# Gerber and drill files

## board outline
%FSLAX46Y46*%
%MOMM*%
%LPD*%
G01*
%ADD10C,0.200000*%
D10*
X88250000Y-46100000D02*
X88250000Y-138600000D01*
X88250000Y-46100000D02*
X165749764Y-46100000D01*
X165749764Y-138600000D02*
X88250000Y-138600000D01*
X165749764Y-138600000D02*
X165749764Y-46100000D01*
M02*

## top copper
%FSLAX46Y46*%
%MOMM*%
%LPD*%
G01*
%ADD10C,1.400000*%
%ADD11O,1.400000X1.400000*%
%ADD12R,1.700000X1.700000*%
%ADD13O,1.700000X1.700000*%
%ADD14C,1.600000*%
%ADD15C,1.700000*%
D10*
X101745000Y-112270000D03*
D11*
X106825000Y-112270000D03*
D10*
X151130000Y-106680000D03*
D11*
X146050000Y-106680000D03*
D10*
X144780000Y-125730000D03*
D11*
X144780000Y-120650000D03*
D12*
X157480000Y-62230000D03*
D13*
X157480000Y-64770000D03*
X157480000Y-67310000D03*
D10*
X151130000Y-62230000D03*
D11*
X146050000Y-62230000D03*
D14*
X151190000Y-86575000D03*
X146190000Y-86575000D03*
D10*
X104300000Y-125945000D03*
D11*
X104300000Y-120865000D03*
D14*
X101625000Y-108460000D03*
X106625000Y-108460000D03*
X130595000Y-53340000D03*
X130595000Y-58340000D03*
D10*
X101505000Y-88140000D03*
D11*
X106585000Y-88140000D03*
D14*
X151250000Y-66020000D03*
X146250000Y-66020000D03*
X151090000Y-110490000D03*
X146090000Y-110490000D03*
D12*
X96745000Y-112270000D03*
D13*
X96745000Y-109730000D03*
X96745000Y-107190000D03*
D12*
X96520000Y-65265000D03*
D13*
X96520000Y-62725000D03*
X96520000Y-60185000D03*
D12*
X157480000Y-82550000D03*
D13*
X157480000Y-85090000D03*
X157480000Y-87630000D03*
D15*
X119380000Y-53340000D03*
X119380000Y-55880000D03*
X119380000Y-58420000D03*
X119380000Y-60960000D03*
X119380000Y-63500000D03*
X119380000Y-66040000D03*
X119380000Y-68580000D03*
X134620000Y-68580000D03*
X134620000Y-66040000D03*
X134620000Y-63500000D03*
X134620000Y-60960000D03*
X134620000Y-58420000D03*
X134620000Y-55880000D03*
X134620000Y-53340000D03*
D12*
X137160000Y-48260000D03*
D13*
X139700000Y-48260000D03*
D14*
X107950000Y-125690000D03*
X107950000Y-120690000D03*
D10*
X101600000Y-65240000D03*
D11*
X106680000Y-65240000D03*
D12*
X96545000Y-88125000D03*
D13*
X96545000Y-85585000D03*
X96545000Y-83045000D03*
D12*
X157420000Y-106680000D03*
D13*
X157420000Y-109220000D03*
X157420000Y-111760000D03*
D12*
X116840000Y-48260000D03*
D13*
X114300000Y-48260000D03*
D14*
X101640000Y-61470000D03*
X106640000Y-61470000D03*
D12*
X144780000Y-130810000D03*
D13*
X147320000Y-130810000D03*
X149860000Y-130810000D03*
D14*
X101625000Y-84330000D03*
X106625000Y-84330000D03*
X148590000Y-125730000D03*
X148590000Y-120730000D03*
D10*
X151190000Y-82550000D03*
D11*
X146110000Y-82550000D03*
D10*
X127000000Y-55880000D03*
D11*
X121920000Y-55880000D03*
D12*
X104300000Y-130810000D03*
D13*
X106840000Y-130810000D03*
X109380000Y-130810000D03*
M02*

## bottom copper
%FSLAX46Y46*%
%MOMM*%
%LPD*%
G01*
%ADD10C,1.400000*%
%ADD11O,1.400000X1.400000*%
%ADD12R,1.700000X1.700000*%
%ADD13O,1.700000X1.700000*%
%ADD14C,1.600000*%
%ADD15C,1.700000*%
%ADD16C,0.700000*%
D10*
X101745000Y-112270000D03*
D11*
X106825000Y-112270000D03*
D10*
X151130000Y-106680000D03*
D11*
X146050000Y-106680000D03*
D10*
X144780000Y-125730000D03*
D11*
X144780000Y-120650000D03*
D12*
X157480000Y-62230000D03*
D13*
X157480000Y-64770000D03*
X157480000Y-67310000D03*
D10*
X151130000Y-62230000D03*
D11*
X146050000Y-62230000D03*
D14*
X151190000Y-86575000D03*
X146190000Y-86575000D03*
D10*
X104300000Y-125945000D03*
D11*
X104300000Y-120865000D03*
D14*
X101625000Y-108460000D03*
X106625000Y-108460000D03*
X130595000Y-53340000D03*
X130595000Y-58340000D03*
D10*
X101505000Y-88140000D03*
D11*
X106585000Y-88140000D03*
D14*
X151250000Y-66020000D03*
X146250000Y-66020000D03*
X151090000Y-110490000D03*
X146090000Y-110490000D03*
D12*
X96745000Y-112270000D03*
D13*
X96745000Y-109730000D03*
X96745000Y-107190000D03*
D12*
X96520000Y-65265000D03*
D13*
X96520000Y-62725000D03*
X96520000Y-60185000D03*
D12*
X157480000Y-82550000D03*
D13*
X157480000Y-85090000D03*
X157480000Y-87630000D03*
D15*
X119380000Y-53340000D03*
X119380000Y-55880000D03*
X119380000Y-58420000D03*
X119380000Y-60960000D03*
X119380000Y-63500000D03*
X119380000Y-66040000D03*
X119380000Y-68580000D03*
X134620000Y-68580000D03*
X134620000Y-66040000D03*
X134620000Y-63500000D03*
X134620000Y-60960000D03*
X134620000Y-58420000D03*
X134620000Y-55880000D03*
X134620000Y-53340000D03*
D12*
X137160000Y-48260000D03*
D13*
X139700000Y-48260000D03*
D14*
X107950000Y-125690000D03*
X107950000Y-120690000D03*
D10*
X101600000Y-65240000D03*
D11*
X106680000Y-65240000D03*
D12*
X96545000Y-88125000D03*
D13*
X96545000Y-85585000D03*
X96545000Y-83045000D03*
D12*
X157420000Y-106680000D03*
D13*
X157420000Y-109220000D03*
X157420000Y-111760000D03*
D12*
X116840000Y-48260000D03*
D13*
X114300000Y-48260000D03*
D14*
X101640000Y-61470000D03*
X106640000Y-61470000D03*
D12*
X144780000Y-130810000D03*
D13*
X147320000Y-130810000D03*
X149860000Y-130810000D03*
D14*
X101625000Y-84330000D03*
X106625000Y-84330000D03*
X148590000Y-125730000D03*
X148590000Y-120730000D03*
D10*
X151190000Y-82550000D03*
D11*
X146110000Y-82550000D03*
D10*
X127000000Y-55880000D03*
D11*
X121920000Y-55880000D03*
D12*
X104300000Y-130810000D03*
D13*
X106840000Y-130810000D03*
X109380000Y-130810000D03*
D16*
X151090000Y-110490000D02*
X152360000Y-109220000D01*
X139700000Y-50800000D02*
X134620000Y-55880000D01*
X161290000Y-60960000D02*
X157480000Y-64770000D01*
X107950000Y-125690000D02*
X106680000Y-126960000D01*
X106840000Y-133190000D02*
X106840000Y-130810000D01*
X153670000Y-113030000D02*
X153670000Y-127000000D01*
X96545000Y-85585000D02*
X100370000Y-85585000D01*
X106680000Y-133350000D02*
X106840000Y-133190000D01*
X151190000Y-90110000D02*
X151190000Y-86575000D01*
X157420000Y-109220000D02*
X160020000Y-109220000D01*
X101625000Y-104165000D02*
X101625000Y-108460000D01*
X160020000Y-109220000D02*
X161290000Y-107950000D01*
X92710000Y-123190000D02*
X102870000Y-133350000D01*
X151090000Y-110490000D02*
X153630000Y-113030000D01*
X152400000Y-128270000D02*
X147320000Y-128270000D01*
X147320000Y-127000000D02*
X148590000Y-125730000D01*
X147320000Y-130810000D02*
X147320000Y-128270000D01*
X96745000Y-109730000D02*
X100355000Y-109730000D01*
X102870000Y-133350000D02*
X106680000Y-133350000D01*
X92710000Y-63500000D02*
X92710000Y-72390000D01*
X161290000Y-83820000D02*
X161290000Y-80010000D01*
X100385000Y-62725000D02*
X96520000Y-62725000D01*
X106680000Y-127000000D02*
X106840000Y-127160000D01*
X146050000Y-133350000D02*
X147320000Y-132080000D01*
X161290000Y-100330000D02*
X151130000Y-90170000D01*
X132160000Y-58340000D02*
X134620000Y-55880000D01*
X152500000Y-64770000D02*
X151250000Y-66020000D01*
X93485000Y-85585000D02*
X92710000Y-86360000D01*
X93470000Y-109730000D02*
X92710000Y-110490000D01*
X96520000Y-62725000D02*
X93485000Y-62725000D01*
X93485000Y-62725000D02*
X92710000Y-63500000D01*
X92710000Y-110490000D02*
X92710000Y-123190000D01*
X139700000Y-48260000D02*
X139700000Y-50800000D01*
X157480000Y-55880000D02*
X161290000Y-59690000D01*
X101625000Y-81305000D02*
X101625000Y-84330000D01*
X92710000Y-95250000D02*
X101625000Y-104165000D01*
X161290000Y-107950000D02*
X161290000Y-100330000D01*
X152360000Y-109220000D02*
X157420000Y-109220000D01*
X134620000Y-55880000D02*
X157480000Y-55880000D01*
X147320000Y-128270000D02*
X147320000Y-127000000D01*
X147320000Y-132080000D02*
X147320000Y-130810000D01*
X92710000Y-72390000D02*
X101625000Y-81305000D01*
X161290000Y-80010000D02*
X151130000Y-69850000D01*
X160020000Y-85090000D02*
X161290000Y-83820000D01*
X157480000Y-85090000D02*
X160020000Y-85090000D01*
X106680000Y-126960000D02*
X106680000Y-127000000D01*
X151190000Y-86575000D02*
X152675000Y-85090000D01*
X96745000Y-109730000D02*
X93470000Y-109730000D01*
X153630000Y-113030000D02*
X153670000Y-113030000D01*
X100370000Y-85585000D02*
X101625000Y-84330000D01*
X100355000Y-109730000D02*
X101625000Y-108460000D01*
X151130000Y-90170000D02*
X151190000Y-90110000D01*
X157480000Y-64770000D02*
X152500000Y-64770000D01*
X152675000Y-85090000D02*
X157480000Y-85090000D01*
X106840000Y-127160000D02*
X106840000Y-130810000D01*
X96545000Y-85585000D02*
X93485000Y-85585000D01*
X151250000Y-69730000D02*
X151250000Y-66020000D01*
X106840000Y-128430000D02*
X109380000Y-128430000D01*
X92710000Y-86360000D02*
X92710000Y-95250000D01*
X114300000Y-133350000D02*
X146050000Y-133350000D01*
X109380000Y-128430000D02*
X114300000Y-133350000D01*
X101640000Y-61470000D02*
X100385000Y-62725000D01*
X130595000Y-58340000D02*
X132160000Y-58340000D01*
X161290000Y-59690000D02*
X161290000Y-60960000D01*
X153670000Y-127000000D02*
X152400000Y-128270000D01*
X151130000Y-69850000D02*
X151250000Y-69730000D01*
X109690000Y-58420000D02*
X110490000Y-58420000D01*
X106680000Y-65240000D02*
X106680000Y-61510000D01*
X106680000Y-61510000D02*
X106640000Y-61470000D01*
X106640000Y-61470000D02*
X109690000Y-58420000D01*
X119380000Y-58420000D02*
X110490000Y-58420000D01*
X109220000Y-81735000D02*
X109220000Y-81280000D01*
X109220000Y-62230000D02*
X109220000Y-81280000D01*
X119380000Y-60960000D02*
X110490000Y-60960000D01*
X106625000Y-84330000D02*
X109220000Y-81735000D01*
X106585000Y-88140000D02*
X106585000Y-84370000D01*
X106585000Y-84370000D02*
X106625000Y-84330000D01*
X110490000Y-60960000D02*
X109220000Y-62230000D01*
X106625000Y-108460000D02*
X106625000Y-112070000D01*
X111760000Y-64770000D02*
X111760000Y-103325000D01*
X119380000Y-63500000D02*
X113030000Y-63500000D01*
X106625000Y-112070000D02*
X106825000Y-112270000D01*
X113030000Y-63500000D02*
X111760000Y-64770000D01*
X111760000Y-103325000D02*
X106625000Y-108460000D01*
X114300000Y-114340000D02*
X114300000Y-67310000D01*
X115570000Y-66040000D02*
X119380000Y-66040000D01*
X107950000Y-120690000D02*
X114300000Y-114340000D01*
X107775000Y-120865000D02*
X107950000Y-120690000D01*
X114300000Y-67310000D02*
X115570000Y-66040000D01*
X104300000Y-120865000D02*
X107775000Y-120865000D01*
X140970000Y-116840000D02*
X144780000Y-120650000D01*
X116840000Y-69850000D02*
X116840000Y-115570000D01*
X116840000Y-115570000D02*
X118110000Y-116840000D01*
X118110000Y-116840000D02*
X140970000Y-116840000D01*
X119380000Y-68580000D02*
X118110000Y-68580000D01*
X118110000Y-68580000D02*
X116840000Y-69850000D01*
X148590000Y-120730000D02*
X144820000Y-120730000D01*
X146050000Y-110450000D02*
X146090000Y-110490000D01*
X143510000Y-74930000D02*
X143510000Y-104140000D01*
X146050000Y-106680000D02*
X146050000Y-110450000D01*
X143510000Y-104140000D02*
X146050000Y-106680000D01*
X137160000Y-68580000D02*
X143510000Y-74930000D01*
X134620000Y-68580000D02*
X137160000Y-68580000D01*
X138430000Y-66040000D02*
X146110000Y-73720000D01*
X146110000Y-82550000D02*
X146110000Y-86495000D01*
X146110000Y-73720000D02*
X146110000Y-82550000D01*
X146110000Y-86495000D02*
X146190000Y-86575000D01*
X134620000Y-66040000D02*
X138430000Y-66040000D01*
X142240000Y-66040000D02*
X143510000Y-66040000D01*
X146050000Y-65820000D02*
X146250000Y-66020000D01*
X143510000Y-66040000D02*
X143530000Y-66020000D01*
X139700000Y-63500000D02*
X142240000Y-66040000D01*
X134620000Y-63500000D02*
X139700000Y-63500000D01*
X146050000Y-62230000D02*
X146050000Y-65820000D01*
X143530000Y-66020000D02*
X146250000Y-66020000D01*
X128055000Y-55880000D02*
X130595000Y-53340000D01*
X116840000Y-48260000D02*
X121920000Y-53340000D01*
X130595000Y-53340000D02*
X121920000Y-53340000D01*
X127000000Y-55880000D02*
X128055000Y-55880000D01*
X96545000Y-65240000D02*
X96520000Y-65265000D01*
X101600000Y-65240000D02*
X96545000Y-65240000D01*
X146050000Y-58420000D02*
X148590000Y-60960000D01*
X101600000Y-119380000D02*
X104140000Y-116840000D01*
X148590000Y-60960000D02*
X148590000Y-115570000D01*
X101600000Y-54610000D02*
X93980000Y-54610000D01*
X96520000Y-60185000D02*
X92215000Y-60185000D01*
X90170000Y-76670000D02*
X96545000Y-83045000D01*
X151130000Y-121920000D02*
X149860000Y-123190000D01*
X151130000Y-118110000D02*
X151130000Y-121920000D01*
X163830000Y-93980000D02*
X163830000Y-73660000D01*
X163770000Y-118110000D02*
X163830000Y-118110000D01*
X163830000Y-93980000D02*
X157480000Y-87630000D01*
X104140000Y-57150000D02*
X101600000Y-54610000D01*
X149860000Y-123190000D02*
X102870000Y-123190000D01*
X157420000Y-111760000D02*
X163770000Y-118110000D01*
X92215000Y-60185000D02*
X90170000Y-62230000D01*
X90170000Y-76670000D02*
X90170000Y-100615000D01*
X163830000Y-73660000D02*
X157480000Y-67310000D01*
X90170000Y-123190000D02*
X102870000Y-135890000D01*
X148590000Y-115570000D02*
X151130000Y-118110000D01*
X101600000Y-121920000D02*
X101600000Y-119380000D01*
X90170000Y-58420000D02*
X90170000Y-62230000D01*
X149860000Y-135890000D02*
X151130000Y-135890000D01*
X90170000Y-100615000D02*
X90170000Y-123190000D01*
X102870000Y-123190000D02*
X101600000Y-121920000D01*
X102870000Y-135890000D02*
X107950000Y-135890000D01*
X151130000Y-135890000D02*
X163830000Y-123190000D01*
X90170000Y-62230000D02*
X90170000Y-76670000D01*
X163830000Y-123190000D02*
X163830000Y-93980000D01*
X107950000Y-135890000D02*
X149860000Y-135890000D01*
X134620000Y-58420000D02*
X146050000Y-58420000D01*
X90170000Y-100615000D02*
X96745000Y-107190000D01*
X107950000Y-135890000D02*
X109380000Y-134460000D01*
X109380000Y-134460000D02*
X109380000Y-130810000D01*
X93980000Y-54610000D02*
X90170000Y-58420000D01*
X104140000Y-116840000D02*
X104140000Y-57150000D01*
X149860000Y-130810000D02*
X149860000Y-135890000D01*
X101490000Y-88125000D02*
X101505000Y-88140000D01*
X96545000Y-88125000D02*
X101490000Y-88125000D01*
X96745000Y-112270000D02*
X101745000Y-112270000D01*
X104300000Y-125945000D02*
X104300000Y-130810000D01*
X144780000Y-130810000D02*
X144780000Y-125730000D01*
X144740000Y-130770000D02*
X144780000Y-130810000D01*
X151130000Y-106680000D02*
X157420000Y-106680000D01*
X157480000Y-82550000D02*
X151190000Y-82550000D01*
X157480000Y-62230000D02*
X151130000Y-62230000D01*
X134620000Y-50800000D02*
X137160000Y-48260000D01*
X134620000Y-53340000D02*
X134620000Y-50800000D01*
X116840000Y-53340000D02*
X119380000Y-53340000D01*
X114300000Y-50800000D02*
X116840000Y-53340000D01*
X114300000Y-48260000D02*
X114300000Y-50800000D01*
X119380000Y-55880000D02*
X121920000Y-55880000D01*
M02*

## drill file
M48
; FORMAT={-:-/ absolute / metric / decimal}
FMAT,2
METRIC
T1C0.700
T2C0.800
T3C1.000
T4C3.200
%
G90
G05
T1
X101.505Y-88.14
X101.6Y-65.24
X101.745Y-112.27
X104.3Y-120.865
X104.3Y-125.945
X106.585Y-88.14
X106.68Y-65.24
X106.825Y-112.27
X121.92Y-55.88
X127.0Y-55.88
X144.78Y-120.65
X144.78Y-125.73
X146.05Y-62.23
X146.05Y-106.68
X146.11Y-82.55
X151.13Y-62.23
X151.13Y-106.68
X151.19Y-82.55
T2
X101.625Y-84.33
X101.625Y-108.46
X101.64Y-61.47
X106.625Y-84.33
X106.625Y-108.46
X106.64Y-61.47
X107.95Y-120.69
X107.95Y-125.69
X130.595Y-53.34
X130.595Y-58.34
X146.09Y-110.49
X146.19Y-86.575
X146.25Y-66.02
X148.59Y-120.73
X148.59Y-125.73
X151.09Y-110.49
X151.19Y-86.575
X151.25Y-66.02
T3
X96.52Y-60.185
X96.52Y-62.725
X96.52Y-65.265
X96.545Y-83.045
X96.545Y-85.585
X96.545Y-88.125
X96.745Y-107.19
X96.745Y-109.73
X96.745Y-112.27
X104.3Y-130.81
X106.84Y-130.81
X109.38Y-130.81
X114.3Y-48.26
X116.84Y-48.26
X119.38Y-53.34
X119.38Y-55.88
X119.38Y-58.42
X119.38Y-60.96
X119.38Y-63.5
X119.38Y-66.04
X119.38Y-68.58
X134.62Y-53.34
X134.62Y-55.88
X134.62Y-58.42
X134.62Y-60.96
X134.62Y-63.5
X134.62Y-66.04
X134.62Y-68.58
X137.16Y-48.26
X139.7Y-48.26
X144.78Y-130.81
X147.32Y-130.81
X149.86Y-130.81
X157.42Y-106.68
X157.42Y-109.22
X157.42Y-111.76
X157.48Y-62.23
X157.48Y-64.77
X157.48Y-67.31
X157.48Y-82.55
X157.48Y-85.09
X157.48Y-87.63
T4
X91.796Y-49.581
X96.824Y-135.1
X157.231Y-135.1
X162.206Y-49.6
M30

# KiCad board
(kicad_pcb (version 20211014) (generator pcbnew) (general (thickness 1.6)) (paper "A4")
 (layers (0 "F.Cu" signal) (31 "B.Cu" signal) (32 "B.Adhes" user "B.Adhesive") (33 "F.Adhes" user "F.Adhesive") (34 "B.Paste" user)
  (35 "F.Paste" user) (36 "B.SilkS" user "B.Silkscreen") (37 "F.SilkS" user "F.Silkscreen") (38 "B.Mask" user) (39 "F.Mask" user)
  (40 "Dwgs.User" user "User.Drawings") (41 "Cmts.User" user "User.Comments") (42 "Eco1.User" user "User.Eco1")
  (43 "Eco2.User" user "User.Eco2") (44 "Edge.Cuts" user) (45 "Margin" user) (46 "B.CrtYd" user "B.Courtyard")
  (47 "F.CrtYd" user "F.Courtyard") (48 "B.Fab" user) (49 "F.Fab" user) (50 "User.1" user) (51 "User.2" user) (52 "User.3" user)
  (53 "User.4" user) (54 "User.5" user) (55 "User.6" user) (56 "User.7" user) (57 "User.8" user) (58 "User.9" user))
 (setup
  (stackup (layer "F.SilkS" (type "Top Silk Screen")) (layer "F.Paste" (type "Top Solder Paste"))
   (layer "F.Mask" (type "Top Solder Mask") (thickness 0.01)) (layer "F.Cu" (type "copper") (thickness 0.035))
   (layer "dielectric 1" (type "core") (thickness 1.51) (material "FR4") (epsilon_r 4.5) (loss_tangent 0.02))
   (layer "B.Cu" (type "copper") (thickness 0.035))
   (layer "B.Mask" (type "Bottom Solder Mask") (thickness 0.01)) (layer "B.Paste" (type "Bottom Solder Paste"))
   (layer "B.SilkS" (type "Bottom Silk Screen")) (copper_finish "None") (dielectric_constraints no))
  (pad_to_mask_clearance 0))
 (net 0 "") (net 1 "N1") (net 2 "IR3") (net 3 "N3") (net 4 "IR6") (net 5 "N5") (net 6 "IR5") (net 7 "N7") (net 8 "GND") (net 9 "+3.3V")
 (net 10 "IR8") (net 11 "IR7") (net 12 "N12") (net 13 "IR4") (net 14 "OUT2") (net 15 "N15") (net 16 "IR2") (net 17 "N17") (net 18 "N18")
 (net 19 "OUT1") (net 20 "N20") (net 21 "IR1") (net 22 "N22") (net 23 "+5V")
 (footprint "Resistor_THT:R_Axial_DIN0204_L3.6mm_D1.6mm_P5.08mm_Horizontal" (layer "F.Cu") (at 101.745 112.27)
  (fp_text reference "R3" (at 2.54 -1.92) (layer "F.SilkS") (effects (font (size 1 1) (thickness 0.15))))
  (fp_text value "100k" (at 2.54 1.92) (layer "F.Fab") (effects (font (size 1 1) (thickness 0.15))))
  (pad "1" thru_hole circle (at 0 0) (size 1.4 1.4) (drill 0.7) (layers *.Cu *.Mask) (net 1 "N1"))
  (pad "2" thru_hole oval (at 5.08 0) (size 1.4 1.4) (drill 0.7) (layers *.Cu *.Mask) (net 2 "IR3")))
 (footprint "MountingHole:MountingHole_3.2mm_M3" (layer "F.Cu") (at 157.231494 135.100002)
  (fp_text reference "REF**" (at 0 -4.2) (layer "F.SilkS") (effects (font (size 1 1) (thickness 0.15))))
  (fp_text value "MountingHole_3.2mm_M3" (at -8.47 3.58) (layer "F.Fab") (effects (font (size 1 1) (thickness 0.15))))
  (pad "" np_thru_hole circle (at 0 0) (size 3.2 3.2) (drill 3.2) (layers F&B.Cu *.Mask)))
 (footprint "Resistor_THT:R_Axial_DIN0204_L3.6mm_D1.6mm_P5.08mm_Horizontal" (layer "F.Cu") (at 151.13 106.68 180)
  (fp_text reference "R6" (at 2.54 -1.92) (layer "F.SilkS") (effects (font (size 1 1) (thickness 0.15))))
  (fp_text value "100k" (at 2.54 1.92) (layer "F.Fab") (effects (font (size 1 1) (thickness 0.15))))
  (pad "1" thru_hole circle (at 0 0 180) (size 1.4 1.4) (drill 0.7) (layers *.Cu *.Mask) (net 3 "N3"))
  (pad "2" thru_hole oval (at 5.08 0 180) (size 1.4 1.4) (drill 0.7) (layers *.Cu *.Mask) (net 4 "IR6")))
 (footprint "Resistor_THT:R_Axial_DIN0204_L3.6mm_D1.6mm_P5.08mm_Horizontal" (layer "F.Cu") (at 144.78 125.73 90)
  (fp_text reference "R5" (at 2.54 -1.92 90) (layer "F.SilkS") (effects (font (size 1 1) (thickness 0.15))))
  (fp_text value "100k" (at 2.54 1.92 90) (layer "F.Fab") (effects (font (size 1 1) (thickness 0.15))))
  (pad "1" thru_hole circle (at 0 0 90) (size 1.4 1.4) (drill 0.7) (layers *.Cu *.Mask) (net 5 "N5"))
  (pad "2" thru_hole oval (at 5.08 0 90) (size 1.4 1.4) (drill 0.7) (layers *.Cu *.Mask) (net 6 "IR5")))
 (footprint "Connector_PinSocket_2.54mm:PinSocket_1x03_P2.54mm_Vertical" (layer "F.Cu") (at 157.48 62.23)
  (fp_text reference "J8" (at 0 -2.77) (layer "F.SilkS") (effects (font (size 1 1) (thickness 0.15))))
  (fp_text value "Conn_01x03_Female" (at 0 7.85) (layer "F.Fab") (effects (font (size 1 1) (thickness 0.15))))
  (pad "1" thru_hole rect (at 0 0) (size 1.7 1.7) (drill 1) (layers *.Cu *.Mask) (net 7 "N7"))
  (pad "2" thru_hole oval (at 0 2.54) (size 1.7 1.7) (drill 1) (layers *.Cu *.Mask) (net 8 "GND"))
  (pad "3" thru_hole oval (at 0 5.08) (size 1.7 1.7) (drill 1) (layers *.Cu *.Mask) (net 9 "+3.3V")))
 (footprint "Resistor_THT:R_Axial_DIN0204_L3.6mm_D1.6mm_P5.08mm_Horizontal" (layer "F.Cu") (at 151.13 62.23 180)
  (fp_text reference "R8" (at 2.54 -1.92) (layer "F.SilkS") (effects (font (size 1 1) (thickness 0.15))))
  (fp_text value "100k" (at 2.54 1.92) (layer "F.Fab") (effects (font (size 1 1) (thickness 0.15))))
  (pad "1" thru_hole circle (at 0 0 180) (size 1.4 1.4) (drill 0.7) (layers *.Cu *.Mask) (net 7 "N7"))
  (pad "2" thru_hole oval (at 5.08 0 180) (size 1.4 1.4) (drill 0.7) (layers *.Cu *.Mask) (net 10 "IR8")))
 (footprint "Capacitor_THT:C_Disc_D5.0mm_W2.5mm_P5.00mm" (layer "F.Cu") (at 151.19 86.575 180)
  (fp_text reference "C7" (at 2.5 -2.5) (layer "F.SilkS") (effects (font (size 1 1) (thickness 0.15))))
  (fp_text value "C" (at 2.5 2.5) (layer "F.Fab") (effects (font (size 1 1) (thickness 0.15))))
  (pad "1" thru_hole circle (at 0 0 180) (size 1.6 1.6) (drill 0.8) (layers *.Cu *.Mask) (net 8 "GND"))
  (pad "2" thru_hole circle (at 5 0 180) (size 1.6 1.6) (drill 0.8) (layers *.Cu *.Mask) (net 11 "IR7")))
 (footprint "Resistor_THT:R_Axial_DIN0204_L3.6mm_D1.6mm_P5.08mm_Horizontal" (layer "F.Cu") (at 104.3 125.945 90)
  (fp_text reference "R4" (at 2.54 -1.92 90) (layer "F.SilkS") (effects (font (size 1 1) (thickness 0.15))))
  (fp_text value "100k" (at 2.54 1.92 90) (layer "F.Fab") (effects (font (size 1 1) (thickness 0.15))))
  (pad "1" thru_hole circle (at 0 0 90) (size 1.4 1.4) (drill 0.7) (layers *.Cu *.Mask) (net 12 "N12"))
  (pad "2" thru_hole oval (at 5.08 0 90) (size 1.4 1.4) (drill 0.7) (layers *.Cu *.Mask) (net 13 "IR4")))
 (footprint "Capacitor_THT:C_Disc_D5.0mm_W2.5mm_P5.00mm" (layer "F.Cu") (at 101.625 108.46)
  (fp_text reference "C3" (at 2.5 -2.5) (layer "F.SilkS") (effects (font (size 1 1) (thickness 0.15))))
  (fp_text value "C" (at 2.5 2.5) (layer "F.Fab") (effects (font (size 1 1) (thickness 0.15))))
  (pad "1" thru_hole circle (at 0 0) (size 1.6 1.6) (drill 0.8) (layers *.Cu *.Mask) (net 8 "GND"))
  (pad "2" thru_hole circle (at 5 0) (size 1.6 1.6) (drill 0.8) (layers *.Cu *.Mask) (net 2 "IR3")))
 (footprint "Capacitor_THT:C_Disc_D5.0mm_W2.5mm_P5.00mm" (layer "F.Cu") (at 130.595 53.34 -90)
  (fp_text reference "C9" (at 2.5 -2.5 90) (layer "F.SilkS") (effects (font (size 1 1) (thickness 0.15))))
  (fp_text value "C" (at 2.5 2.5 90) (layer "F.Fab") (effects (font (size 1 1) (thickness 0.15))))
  (pad "1" thru_hole circle (at 0 0 270) (size 1.6 1.6) (drill 0.8) (layers *.Cu *.Mask) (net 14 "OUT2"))
  (pad "2" thru_hole circle (at 5 0 270) (size 1.6 1.6) (drill 0.8) (layers *.Cu *.Mask) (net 8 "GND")))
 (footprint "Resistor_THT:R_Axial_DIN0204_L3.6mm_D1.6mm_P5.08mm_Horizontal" (layer "F.Cu") (at 101.505 88.14)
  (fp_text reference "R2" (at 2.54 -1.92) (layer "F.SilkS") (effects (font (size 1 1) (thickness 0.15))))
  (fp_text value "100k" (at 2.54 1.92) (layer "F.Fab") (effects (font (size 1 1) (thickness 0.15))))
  (pad "1" thru_hole circle (at 0 0) (size 1.4 1.4) (drill 0.7) (layers *.Cu *.Mask) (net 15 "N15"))
  (pad "2" thru_hole oval (at 5.08 0) (size 1.4 1.4) (drill 0.7) (layers *.Cu *.Mask) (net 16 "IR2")))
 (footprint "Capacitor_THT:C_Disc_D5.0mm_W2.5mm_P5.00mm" (layer "F.Cu") (at 151.25 66.02 180)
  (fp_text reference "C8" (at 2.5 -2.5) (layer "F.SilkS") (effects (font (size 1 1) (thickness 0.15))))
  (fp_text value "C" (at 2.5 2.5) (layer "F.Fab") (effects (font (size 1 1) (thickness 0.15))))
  (pad "1" thru_hole circle (at 0 0 180) (size 1.6 1.6) (drill 0.8) (layers *.Cu *.Mask) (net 8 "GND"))
  (pad "2" thru_hole circle (at 5 0 180) (size 1.6 1.6) (drill 0.8) (layers *.Cu *.Mask) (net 10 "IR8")))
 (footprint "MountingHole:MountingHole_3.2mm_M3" (layer "F.Cu") (at 162.205882 49.600001)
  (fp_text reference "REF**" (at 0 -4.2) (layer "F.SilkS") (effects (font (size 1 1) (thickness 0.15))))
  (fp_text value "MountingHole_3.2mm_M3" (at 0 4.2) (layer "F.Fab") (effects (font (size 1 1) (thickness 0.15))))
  (pad "" np_thru_hole circle (at 0 0) (size 3.2 3.2) (drill 3.2) (layers F&B.Cu *.Mask)))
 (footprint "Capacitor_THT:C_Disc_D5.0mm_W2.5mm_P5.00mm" (layer "F.Cu") (at 151.09 110.49 180)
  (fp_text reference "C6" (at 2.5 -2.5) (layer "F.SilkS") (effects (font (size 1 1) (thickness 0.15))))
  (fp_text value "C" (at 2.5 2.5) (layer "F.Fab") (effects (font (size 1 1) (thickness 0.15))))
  (pad "1" thru_hole circle (at 0 0 180) (size 1.6 1.6) (drill 0.8) (layers *.Cu *.Mask) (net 8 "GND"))
  (pad "2" thru_hole circle (at 5 0 180) (size 1.6 1.6) (drill 0.8) (layers *.Cu *.Mask) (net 4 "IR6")))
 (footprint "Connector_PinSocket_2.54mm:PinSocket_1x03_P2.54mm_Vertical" (layer "F.Cu") (at 96.745 112.27 180)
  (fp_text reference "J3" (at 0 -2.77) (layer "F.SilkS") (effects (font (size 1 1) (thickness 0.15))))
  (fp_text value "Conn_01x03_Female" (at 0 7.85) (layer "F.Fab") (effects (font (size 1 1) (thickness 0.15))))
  (pad "1" thru_hole rect (at 0 0 180) (size 1.7 1.7) (drill 1) (layers *.Cu *.Mask) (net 1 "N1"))
  (pad "2" thru_hole oval (at 0 2.54 180) (size 1.7 1.7) (drill 1) (layers *.Cu *.Mask) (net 8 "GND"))
  (pad "3" thru_hole oval (at 0 5.08 180) (size 1.7 1.7) (drill 1) (layers *.Cu *.Mask) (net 9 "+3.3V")))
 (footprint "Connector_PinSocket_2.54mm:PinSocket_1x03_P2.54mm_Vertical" (layer "F.Cu") (at 96.52 65.265 180)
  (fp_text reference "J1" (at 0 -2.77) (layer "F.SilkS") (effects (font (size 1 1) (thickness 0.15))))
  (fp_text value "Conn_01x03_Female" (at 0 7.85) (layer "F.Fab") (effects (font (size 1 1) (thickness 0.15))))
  (pad "1" thru_hole rect (at 0 0 180) (size 1.7 1.7) (drill 1) (layers *.Cu *.Mask) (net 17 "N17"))
  (pad "2" thru_hole oval (at 0 2.54 180) (size 1.7 1.7) (drill 1) (layers *.Cu *.Mask) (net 8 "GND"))
  (pad "3" thru_hole oval (at 0 5.08 180) (size 1.7 1.7) (drill 1) (layers *.Cu *.Mask) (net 9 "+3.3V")))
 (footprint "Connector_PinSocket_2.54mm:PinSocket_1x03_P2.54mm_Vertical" (layer "F.Cu") (at 157.48 82.55)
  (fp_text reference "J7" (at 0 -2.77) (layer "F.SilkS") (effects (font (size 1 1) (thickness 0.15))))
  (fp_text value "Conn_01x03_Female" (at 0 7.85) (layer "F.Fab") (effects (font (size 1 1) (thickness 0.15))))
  (pad "1" thru_hole rect (at 0 0) (size 1.7 1.7) (drill 1) (layers *.Cu *.Mask) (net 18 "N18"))
  (pad "2" thru_hole oval (at 0 2.54) (size 1.7 1.7) (drill 1) (layers *.Cu *.Mask) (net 8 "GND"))
  (pad "3" thru_hole oval (at 0 5.08) (size 1.7 1.7) (drill 1) (layers *.Cu *.Mask) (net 9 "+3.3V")))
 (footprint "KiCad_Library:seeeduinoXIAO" (layer "F.Cu") (at 127 60.96 180)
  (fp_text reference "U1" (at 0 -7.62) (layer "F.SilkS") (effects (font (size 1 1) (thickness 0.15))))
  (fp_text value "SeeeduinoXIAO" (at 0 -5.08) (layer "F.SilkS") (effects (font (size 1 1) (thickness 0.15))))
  (pad "1" thru_hole circle (at 7.62 7.62 180) (size 1.7 1.7) (drill 1) (layers *.Cu *.Mask) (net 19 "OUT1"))
  (pad "2" thru_hole circle (at 7.62 5.08 180) (size 1.7 1.7) (drill 1) (layers *.Cu *.Mask) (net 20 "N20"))
  (pad "3" thru_hole circle (at 7.62 2.54 180) (size 1.7 1.7) (drill 1) (layers *.Cu *.Mask) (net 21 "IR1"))
  (pad "4" thru_hole circle (at 7.62 0 180) (size 1.7 1.7) (drill 1) (layers *.Cu *.Mask) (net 16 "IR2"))
  (pad "5" thru_hole circle (at 7.62 -2.54 180) (size 1.7 1.7) (drill 1) (layers *.Cu *.Mask) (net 2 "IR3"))
  (pad "6" thru_hole circle (at 7.62 -5.08 180) (size 1.7 1.7) (drill 1) (layers *.Cu *.Mask) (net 13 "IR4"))
  (pad "7" thru_hole circle (at 7.62 -7.62 180) (size 1.7 1.7) (drill 1) (layers *.Cu *.Mask) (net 6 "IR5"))
  (pad "8" thru_hole circle (at -7.62 -7.62 180) (size 1.7 1.7) (drill 1) (layers *.Cu *.Mask) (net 4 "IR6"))
  (pad "9" thru_hole circle (at -7.62 -5.08 180) (size 1.7 1.7) (drill 1) (layers *.Cu *.Mask) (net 11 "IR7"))
  (pad "10" thru_hole circle (at -7.62 -2.54 180) (size 1.7 1.7) (drill 1) (layers *.Cu *.Mask) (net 10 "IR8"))
  (pad "11" thru_hole circle (at -7.62 0 180) (size 1.7 1.7) (drill 1) (layers *.Cu *.Mask) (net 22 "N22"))
  (pad "12" thru_hole circle (at -7.62 2.54 180) (size 1.7 1.7) (drill 1) (layers *.Cu *.Mask) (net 9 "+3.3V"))
  (pad "13" thru_hole circle (at -7.62 5.08 180) (size 1.7 1.7) (drill 1) (layers *.Cu *.Mask) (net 8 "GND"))
  (pad "14" thru_hole circle (at -7.62 7.62 180) (size 1.7 1.7) (drill 1) (layers *.Cu *.Mask) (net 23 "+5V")))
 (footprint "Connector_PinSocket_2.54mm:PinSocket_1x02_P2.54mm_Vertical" (layer "F.Cu") (at 137.16 48.26 90)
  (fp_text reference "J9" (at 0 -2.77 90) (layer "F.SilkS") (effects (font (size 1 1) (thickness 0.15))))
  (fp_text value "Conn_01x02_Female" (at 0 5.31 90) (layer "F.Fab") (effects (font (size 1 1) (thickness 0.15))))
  (pad "1" thru_hole rect (at 0 0 90) (size 1.7 1.7) (drill 1) (layers *.Cu *.Mask) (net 23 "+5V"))
  (pad "2" thru_hole oval (at 0 2.54 90) (size 1.7 1.7) (drill 1) (layers *.Cu *.Mask) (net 8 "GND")))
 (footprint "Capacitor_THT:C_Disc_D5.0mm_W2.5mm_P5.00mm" (layer "F.Cu") (at 107.95 125.69 90)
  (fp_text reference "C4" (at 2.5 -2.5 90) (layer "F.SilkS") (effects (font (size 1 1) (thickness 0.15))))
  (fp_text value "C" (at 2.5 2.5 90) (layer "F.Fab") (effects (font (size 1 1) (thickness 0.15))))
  (pad "1" thru_hole circle (at 0 0 90) (size 1.6 1.6) (drill 0.8) (layers *.Cu *.Mask) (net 8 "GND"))
  (pad "2" thru_hole circle (at 5 0 90) (size 1.6 1.6) (drill 0.8) (layers *.Cu *.Mask) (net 13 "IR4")))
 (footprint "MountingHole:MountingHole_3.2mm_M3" (layer "F.Cu") (at 91.7956 49.5808)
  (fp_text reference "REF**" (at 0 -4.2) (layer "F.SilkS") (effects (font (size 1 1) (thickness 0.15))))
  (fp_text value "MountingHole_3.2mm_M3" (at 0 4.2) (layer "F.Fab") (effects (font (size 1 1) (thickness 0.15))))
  (pad "" np_thru_hole circle (at 0 0) (size 3.2 3.2) (drill 3.2) (layers *.Cu *.Mask)))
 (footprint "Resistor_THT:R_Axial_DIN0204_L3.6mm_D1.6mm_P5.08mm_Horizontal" (layer "F.Cu") (at 101.6 65.24)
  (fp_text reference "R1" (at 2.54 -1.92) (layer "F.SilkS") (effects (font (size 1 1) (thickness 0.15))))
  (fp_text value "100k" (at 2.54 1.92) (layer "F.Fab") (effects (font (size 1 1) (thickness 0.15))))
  (pad "1" thru_hole circle (at 0 0) (size 1.4 1.4) (drill 0.7) (layers *.Cu *.Mask) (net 17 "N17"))
  (pad "2" thru_hole oval (at 5.08 0) (size 1.4 1.4) (drill 0.7) (layers *.Cu *.Mask) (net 21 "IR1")))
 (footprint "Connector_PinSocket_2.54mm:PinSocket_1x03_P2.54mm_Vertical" (layer "F.Cu") (at 96.545 88.125 180)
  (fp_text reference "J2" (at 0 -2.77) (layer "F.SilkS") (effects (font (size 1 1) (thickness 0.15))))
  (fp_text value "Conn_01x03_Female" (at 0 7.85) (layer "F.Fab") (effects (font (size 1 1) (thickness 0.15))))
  (pad "1" thru_hole rect (at 0 0 180) (size 1.7 1.7) (drill 1) (layers *.Cu *.Mask) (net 15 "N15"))
  (pad "2" thru_hole oval (at 0 2.54 180) (size 1.7 1.7) (drill 1) (layers *.Cu *.Mask) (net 8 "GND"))
  (pad "3" thru_hole oval (at 0 5.08 180) (size 1.7 1.7) (drill 1) (layers *.Cu *.Mask) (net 9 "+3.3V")))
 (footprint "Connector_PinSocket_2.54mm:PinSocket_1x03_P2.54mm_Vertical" (layer "F.Cu") (at 157.42 106.68)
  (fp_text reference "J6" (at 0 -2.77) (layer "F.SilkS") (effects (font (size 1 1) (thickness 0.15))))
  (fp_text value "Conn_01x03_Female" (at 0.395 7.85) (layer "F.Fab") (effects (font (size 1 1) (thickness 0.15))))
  (pad "1" thru_hole rect (at 0 0) (size 1.7 1.7) (drill 1) (layers *.Cu *.Mask) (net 3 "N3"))
  (pad "2" thru_hole oval (at 0 2.54) (size 1.7 1.7) (drill 1) (layers *.Cu *.Mask) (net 8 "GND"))
  (pad "3" thru_hole oval (at 0 5.08) (size 1.7 1.7) (drill 1) (layers *.Cu *.Mask) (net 9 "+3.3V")))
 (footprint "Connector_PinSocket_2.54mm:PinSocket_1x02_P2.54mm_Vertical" (layer "F.Cu") (at 116.84 48.26 -90)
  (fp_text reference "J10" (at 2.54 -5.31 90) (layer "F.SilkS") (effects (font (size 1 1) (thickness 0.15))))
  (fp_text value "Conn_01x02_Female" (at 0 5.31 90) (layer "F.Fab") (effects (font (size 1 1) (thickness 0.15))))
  (pad "1" thru_hole rect (at 0 0 270) (size 1.7 1.7) (drill 1) (layers *.Cu *.Mask) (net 14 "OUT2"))
  (pad "2" thru_hole oval (at 0 2.54 270) (size 1.7 1.7) (drill 1) (layers *.Cu *.Mask) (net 19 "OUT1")))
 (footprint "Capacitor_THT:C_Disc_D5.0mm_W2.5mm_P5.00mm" (layer "F.Cu") (at 101.64 61.47)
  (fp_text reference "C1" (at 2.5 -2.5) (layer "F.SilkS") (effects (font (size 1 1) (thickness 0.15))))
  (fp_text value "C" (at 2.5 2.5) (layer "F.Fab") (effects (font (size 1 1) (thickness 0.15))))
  (pad "1" thru_hole circle (at 0 0) (size 1.6 1.6) (drill 0.8) (layers *.Cu *.Mask) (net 8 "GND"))
  (pad "2" thru_hole circle (at 5 0) (size 1.6 1.6) (drill 0.8) (layers *.Cu *.Mask) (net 21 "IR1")))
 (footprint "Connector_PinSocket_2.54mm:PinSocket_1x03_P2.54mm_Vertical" (layer "F.Cu") (at 144.78 130.81 90)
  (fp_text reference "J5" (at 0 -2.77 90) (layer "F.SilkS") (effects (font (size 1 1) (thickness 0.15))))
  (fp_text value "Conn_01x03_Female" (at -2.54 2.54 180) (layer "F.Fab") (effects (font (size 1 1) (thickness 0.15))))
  (pad "1" thru_hole rect (at 0 0 90) (size 1.7 1.7) (drill 1) (layers *.Cu *.Mask) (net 5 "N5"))
  (pad "2" thru_hole oval (at 0 2.54 90) (size 1.7 1.7) (drill 1) (layers *.Cu *.Mask) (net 8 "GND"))
  (pad "3" thru_hole oval (at 0 5.08 90) (size 1.7 1.7) (drill 1) (layers *.Cu *.Mask) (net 9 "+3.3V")))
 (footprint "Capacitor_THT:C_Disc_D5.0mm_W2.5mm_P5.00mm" (layer "F.Cu") (at 101.625 84.33)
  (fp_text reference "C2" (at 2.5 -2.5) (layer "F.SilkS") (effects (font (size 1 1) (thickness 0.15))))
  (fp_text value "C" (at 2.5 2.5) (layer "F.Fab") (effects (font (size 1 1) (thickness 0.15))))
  (pad "1" thru_hole circle (at 0 0) (size 1.6 1.6) (drill 0.8) (layers *.Cu *.Mask) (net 8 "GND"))
  (pad "2" thru_hole circle (at 5 0) (size 1.6 1.6) (drill 0.8) (layers *.Cu *.Mask) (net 16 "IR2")))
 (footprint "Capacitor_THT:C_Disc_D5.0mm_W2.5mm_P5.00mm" (layer "F.Cu") (at 148.59 125.73 90)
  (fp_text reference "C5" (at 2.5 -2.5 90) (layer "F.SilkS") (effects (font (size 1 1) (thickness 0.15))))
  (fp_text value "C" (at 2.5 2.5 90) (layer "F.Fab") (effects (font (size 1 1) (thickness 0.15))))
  (pad "1" thru_hole circle (at 0 0 90) (size 1.6 1.6) (drill 0.8) (layers *.Cu *.Mask) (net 8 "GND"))
  (pad "2" thru_hole circle (at 5 0 90) (size 1.6 1.6) (drill 0.8) (layers *.Cu *.Mask) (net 6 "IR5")))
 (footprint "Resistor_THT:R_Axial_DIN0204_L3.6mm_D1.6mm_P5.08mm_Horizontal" (layer "F.Cu") (at 151.19 82.55 180)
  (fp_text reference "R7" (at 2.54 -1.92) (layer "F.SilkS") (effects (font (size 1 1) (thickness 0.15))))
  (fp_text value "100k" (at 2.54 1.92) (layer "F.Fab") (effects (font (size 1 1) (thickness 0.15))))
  (pad "1" thru_hole circle (at 0 0 180) (size 1.4 1.4) (drill 0.7) (layers *.Cu *.Mask) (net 18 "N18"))
  (pad "2" thru_hole oval (at 5.08 0 180) (size 1.4 1.4) (drill 0.7) (layers *.Cu *.Mask) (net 11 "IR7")))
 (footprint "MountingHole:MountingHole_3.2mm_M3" (layer "F.Cu") (at 96.82353 135.100002)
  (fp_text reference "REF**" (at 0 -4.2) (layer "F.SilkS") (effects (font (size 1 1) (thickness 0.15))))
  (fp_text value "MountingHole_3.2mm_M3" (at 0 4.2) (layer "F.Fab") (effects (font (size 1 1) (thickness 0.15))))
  (pad "" np_thru_hole circle (at 0 0) (size 3.2 3.2) (drill 3.2) (layers F&B.Cu *.Mask)))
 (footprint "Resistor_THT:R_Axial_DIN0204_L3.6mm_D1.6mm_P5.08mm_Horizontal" (layer "F.Cu") (at 127 55.88 180)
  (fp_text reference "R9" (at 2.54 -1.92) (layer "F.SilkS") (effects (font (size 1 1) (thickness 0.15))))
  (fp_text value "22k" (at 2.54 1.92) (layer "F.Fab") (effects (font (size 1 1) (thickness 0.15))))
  (pad "1" thru_hole circle (at 0 0 180) (size 1.4 1.4) (drill 0.7) (layers *.Cu *.Mask) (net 14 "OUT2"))
  (pad "2" thru_hole oval (at 5.08 0 180) (size 1.4 1.4) (drill 0.7) (layers *.Cu *.Mask) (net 20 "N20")))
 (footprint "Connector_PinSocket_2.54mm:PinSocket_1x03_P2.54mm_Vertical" (layer "F.Cu") (at 104.3 130.81 90)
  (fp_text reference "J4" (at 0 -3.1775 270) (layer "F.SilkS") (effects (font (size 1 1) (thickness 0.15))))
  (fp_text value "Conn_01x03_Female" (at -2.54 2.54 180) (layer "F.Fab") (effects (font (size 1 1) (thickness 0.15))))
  (pad "1" thru_hole rect (at 0 0 90) (size 1.7 1.7) (drill 1) (layers *.Cu *.Mask) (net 12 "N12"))
  (pad "2" thru_hole oval (at 0 2.54 90) (size 1.7 1.7) (drill 1) (layers *.Cu *.Mask) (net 8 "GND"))
  (pad "3" thru_hole oval (at 0 5.08 90) (size 1.7 1.7) (drill 1) (layers *.Cu *.Mask) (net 9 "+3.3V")))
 (gr_line (start 88.25 46.1) (end 88.25 138.6) (layer "Edge.Cuts") (width 0.2))
 (gr_line (start 88.25 46.1) (end 165.749764 46.1) (layer "Edge.Cuts") (width 0.2))
 (gr_line (start 165.749764 138.6) (end 88.25 138.6) (layer "Edge.Cuts") (width 0.2))
 (gr_line (start 165.749764 138.6) (end 165.749764 46.1) (layer "Edge.Cuts") (width 0.2))
 (segment (start 151.09 110.49) (end 152.36 109.22) (width 0.7) (layer "B.Cu") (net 8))
 (segment (start 139.7 50.8) (end 134.62 55.88) (width 0.7) (layer "B.Cu") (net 8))
 (segment (start 161.29 60.96) (end 157.48 64.77) (width 0.7) (layer "B.Cu") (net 8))
 (segment (start 107.95 125.69) (end 106.68 126.96) (width 0.7) (layer "B.Cu") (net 8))
 (segment (start 106.84 133.19) (end 106.84 130.81) (width 0.7) (layer "B.Cu") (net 8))
 (segment (start 153.67 113.03) (end 153.67 127) (width 0.7) (layer "B.Cu") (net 8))
 (segment (start 96.545 85.585) (end 100.37 85.585) (width 0.7) (layer "B.Cu") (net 8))
 (segment (start 106.68 133.35) (end 106.84 133.19) (width 0.7) (layer "B.Cu") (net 8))
 (segment (start 151.19 90.11) (end 151.19 86.575) (width 0.7) (layer "B.Cu") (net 8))
 (segment (start 157.42 109.22) (end 160.02 109.22) (width 0.7) (layer "B.Cu") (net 8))
 (segment (start 101.625 104.165) (end 101.625 108.46) (width 0.7) (layer "B.Cu") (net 8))
 (segment (start 160.02 109.22) (end 161.29 107.95) (width 0.7) (layer "B.Cu") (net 8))
 (segment (start 92.71 123.19) (end 102.87 133.35) (width 0.7) (layer "B.Cu") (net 8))
 (segment (start 151.09 110.49) (end 153.63 113.03) (width 0.7) (layer "B.Cu") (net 8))
 (segment (start 152.4 128.27) (end 147.32 128.27) (width 0.7) (layer "B.Cu") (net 8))
 (segment (start 147.32 127) (end 148.59 125.73) (width 0.7) (layer "B.Cu") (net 8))
 (segment (start 147.32 130.81) (end 147.32 128.27) (width 0.7) (layer "B.Cu") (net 8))
 (segment (start 96.745 109.73) (end 100.355 109.73) (width 0.7) (layer "B.Cu") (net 8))
 (segment (start 102.87 133.35) (end 106.68 133.35) (width 0.7) (layer "B.Cu") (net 8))
 (segment (start 92.71 63.5) (end 92.71 72.39) (width 0.7) (layer "B.Cu") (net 8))
 (segment (start 161.29 83.82) (end 161.29 80.01) (width 0.7) (layer "B.Cu") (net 8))
 (segment (start 100.385 62.725) (end 96.52 62.725) (width 0.7) (layer "B.Cu") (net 8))
 (segment (start 106.68 127) (end 106.84 127.16) (width 0.7) (layer "B.Cu") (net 8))
 (segment (start 146.05 133.35) (end 147.32 132.08) (width 0.7) (layer "B.Cu") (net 8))
 (segment (start 161.29 100.33) (end 151.13 90.17) (width 0.7) (layer "B.Cu") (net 8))
 (segment (start 132.16 58.34) (end 134.62 55.88) (width 0.7) (layer "B.Cu") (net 8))
 (segment (start 152.5 64.77) (end 151.25 66.02) (width 0.7) (layer "B.Cu") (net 8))
 (segment (start 93.485 85.585) (end 92.71 86.36) (width 0.7) (layer "B.Cu") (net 8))
 (segment (start 93.47 109.73) (end 92.71 110.49) (width 0.7) (layer "B.Cu") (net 8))
 (segment (start 96.52 62.725) (end 93.485 62.725) (width 0.7) (layer "B.Cu") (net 8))
 (segment (start 93.485 62.725) (end 92.71 63.5) (width 0.7) (layer "B.Cu") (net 8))
 (segment (start 92.71 110.49) (end 92.71 123.19) (width 0.7) (layer "B.Cu") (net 8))
 (segment (start 139.7 48.26) (end 139.7 50.8) (width 0.7) (layer "B.Cu") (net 8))
 (segment (start 157.48 55.88) (end 161.29 59.69) (width 0.7) (layer "B.Cu") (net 8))
 (segment (start 101.625 81.305) (end 101.625 84.33) (width 0.7) (layer "B.Cu") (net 8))
 (segment (start 92.71 95.25) (end 101.625 104.165) (width 0.7) (layer "B.Cu") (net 8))
 (segment (start 161.29 107.95) (end 161.29 100.33) (width 0.7) (layer "B.Cu") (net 8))
 (segment (start 152.36 109.22) (end 157.42 109.22) (width 0.7) (layer "B.Cu") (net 8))
 (segment (start 134.62 55.88) (end 157.48 55.88) (width 0.7) (layer "B.Cu") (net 8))
 (segment (start 147.32 128.27) (end 147.32 127) (width 0.7) (layer "B.Cu") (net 8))
 (segment (start 147.32 132.08) (end 147.32 130.81) (width 0.7) (layer "B.Cu") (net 8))
 (segment (start 92.71 72.39) (end 101.625 81.305) (width 0.7) (layer "B.Cu") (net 8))
 (segment (start 161.29 80.01) (end 151.13 69.85) (width 0.7) (layer "B.Cu") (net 8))
 (segment (start 160.02 85.09) (end 161.29 83.82) (width 0.7) (layer "B.Cu") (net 8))
 (segment (start 157.48 85.09) (end 160.02 85.09) (width 0.7) (layer "B.Cu") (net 8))
 (segment (start 106.68 126.96) (end 106.68 127) (width 0.7) (layer "B.Cu") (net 8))
 (segment (start 151.19 86.575) (end 152.675 85.09) (width 0.7) (layer "B.Cu") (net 8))
 (segment (start 96.745 109.73) (end 93.47 109.73) (width 0.7) (layer "B.Cu") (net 8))
 (segment (start 153.63 113.03) (end 153.67 113.03) (width 0.7) (layer "B.Cu") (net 8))
 (segment (start 100.37 85.585) (end 101.625 84.33) (width 0.7) (layer "B.Cu") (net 8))
 (segment (start 100.355 109.73) (end 101.625 108.46) (width 0.7) (layer "B.Cu") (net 8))
 (segment (start 151.13 90.17) (end 151.19 90.11) (width 0.7) (layer "B.Cu") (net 8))
 (segment (start 157.48 64.77) (end 152.5 64.77) (width 0.7) (layer "B.Cu") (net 8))
 (segment (start 152.675 85.09) (end 157.48 85.09) (width 0.7) (layer "B.Cu") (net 8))
 (segment (start 106.84 127.16) (end 106.84 130.81) (width 0.7) (layer "B.Cu") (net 8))
 (segment (start 96.545 85.585) (end 93.485 85.585) (width 0.7) (layer "B.Cu") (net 8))
 (segment (start 151.25 69.73) (end 151.25 66.02) (width 0.7) (layer "B.Cu") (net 8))
 (segment (start 106.84 128.43) (end 109.38 128.43) (width 0.7) (layer "B.Cu") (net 8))
 (segment (start 92.71 86.36) (end 92.71 95.25) (width 0.7) (layer "B.Cu") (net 8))
 (segment (start 114.3 133.35) (end 146.05 133.35) (width 0.7) (layer "B.Cu") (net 8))
 (segment (start 109.38 128.43) (end 114.3 133.35) (width 0.7) (layer "B.Cu") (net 8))
 (segment (start 101.64 61.47) (end 100.385 62.725) (width 0.7) (layer "B.Cu") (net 8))
 (segment (start 130.595 58.34) (end 132.16 58.34) (width 0.7) (layer "B.Cu") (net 8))
 (segment (start 161.29 59.69) (end 161.29 60.96) (width 0.7) (layer "B.Cu") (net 8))
 (segment (start 153.67 127) (end 152.4 128.27) (width 0.7) (layer "B.Cu") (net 8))
 (segment (start 151.13 69.85) (end 151.25 69.73) (width 0.7) (layer "B.Cu") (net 8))
 (segment (start 109.69 58.42) (end 110.49 58.42) (width 0.7) (layer "B.Cu") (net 21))
 (segment (start 106.68 65.24) (end 106.68 61.51) (width 0.7) (layer "B.Cu") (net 21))
 (segment (start 106.68 61.51) (end 106.64 61.47) (width 0.7) (layer "B.Cu") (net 21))
 (segment (start 106.64 61.47) (end 109.69 58.42) (width 0.7) (layer "B.Cu") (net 21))
 (segment (start 119.38 58.42) (end 110.49 58.42) (width 0.7) (layer "B.Cu") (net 21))
 (segment (start 109.22 81.735) (end 109.22 81.28) (width 0.7) (layer "B.Cu") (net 16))
 (segment (start 109.22 62.23) (end 109.22 81.28) (width 0.7) (layer "B.Cu") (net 16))
 (segment (start 119.38 60.96) (end 110.49 60.96) (width 0.7) (layer "B.Cu") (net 16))
 (segment (start 106.625 84.33) (end 109.22 81.735) (width 0.7) (layer "B.Cu") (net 16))
 (segment (start 106.585 88.14) (end 106.585 84.37) (width 0.7) (layer "B.Cu") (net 16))
 (segment (start 106.585 84.37) (end 106.625 84.33) (width 0.7) (layer "B.Cu") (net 16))
 (segment (start 110.49 60.96) (end 109.22 62.23) (width 0.7) (layer "B.Cu") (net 16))
 (segment (start 106.625 108.46) (end 106.625 112.07) (width 0.7) (layer "B.Cu") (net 2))
 (segment (start 111.76 64.77) (end 111.76 103.325) (width 0.7) (layer "B.Cu") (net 2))
 (segment (start 119.38 63.5) (end 113.03 63.5) (width 0.7) (layer "B.Cu") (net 2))
 (segment (start 106.625 112.07) (end 106.825 112.27) (width 0.7) (layer "B.Cu") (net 2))
 (segment (start 113.03 63.5) (end 111.76 64.77) (width 0.7) (layer "B.Cu") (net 2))
 (segment (start 111.76 103.325) (end 106.625 108.46) (width 0.7) (layer "B.Cu") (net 2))
 (segment (start 114.3 114.34) (end 114.3 67.31) (width 0.7) (layer "B.Cu") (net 13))
 (segment (start 115.57 66.04) (end 119.38 66.04) (width 0.7) (layer "B.Cu") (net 13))
 (segment (start 107.95 120.69) (end 114.3 114.34) (width 0.7) (layer "B.Cu") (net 13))
 (segment (start 107.775 120.865) (end 107.95 120.69) (width 0.7) (layer "B.Cu") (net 13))
 (segment (start 114.3 67.31) (end 115.57 66.04) (width 0.7) (layer "B.Cu") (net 13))
 (segment (start 104.3 120.865) (end 107.775 120.865) (width 0.7) (layer "B.Cu") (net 13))
 (segment (start 140.97 116.84) (end 144.78 120.65) (width 0.7) (layer "B.Cu") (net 6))
 (segment (start 116.84 69.85) (end 116.84 115.57) (width 0.7) (layer "B.Cu") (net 6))
 (segment (start 116.84 115.57) (end 118.11 116.84) (width 0.7) (layer "B.Cu") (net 6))
 (segment (start 118.11 116.84) (end 140.97 116.84) (width 0.7) (layer "B.Cu") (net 6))
 (segment (start 119.38 68.58) (end 118.11 68.58) (width 0.7) (layer "B.Cu") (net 6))
 (segment (start 118.11 68.58) (end 116.84 69.85) (width 0.7) (layer "B.Cu") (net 6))
 (segment (start 148.59 120.73) (end 144.82 120.73) (width 0.7) (layer "B.Cu") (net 6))
 (segment (start 146.05 110.45) (end 146.09 110.49) (width 0.7) (layer "B.Cu") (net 4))
 (segment (start 143.51 74.93) (end 143.51 104.14) (width 0.7) (layer "B.Cu") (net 4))
 (segment (start 146.05 106.68) (end 146.05 110.45) (width 0.7) (layer "B.Cu") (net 4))
 (segment (start 143.51 104.14) (end 146.05 106.68) (width 0.7) (layer "B.Cu") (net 4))
 (segment (start 137.16 68.58) (end 143.51 74.93) (width 0.7) (layer "B.Cu") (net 4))
 (segment (start 134.62 68.58) (end 137.16 68.58) (width 0.7) (layer "B.Cu") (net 4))
 (segment (start 138.43 66.04) (end 146.11 73.72) (width 0.7) (layer "B.Cu") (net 11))
 (segment (start 146.11 82.55) (end 146.11 86.495) (width 0.7) (layer "B.Cu") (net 11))
 (segment (start 146.11 73.72) (end 146.11 82.55) (width 0.7) (layer "B.Cu") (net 11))
 (segment (start 146.11 86.495) (end 146.19 86.575) (width 0.7) (layer "B.Cu") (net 11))
 (segment (start 134.62 66.04) (end 138.43 66.04) (width 0.7) (layer "B.Cu") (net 11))
 (segment (start 142.24 66.04) (end 143.51 66.04) (width 0.7) (layer "B.Cu") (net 10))
 (segment (start 146.05 65.82) (end 146.25 66.02) (width 0.7) (layer "B.Cu") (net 10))
 (segment (start 143.51 66.04) (end 143.53 66.02) (width 0.7) (layer "B.Cu") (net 10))
 (segment (start 139.7 63.5) (end 142.24 66.04) (width 0.7) (layer "B.Cu") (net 10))
 (segment (start 134.62 63.5) (end 139.7 63.5) (width 0.7) (layer "B.Cu") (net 10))
 (segment (start 146.05 62.23) (end 146.05 65.82) (width 0.7) (layer "B.Cu") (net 10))
 (segment (start 143.53 66.02) (end 146.25 66.02) (width 0.7) (layer "B.Cu") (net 10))
 (segment (start 128.055 55.88) (end 130.595 53.34) (width 0.7) (layer "B.Cu") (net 14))
 (segment (start 116.84 48.26) (end 121.92 53.34) (width 0.7) (layer "B.Cu") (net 14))
 (segment (start 130.595 53.34) (end 121.92 53.34) (width 0.7) (layer "B.Cu") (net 14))
 (segment (start 127 55.88) (end 128.055 55.88) (width 0.7) (layer "B.Cu") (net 14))
 (segment (start 96.545 65.24) (end 96.52 65.265) (width 0.7) (layer "B.Cu") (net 17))
 (segment (start 101.6 65.24) (end 96.545 65.24) (width 0.7) (layer "B.Cu") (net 17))
 (segment (start 146.05 58.42) (end 148.59 60.96) (width 0.7) (layer "B.Cu") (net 9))
 (segment (start 101.6 119.38) (end 104.14 116.84) (width 0.7) (layer "B.Cu") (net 9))
 (segment (start 148.59 60.96) (end 148.59 115.57) (width 0.7) (layer "B.Cu") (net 9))
 (segment (start 101.6 54.61) (end 93.98 54.61) (width 0.7) (layer "B.Cu") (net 9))
 (segment (start 96.52 60.185) (end 92.215 60.185) (width 0.7) (layer "B.Cu") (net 9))
 (segment (start 90.17 76.67) (end 96.545 83.045) (width 0.7) (layer "B.Cu") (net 9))
 (segment (start 151.13 121.92) (end 149.86 123.19) (width 0.7) (layer "B.Cu") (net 9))
 (segment (start 151.13 118.11) (end 151.13 121.92) (width 0.7) (layer "B.Cu") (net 9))
 (segment (start 163.83 93.98) (end 163.83 73.66) (width 0.7) (layer "B.Cu") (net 9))
 (segment (start 163.77 118.11) (end 163.83 118.11) (width 0.7) (layer "B.Cu") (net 9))
 (segment (start 163.83 93.98) (end 157.48 87.63) (width 0.7) (layer "B.Cu") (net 9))
 (segment (start 104.14 57.15) (end 101.6 54.61) (width 0.7) (layer "B.Cu") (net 9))
 (segment (start 149.86 123.19) (end 102.87 123.19) (width 0.7) (layer "B.Cu") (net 9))
 (segment (start 157.42 111.76) (end 163.77 118.11) (width 0.7) (layer "B.Cu") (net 9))
 (segment (start 92.215 60.185) (end 90.17 62.23) (width 0.7) (layer "B.Cu") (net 9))
 (segment (start 90.17 76.67) (end 90.17 100.615) (width 0.7) (layer "B.Cu") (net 9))
 (segment (start 163.83 73.66) (end 157.48 67.31) (width 0.7) (layer "B.Cu") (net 9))
 (segment (start 90.17 123.19) (end 102.87 135.89) (width 0.7) (layer "B.Cu") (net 9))
 (segment (start 148.59 115.57) (end 151.13 118.11) (width 0.7) (layer "B.Cu") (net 9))
 (segment (start 101.6 121.92) (end 101.6 119.38) (width 0.7) (layer "B.Cu") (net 9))
 (segment (start 90.17 58.42) (end 90.17 62.23) (width 0.7) (layer "B.Cu") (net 9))
 (segment (start 149.86 135.89) (end 151.13 135.89) (width 0.7) (layer "B.Cu") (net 9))
 (segment (start 90.17 100.615) (end 90.17 123.19) (width 0.7) (layer "B.Cu") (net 9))
 (segment (start 102.87 123.19) (end 101.6 121.92) (width 0.7) (layer "B.Cu") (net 9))
 (segment (start 102.87 135.89) (end 107.95 135.89) (width 0.7) (layer "B.Cu") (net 9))
 (segment (start 151.13 135.89) (end 163.83 123.19) (width 0.7) (layer "B.Cu") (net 9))
 (segment (start 90.17 62.23) (end 90.17 76.67) (width 0.7) (layer "B.Cu") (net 9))
 (segment (start 163.83 123.19) (end 163.83 93.98) (width 0.7) (layer "B.Cu") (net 9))
 (segment (start 107.95 135.89) (end 149.86 135.89) (width 0.7) (layer "B.Cu") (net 9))
 (segment (start 134.62 58.42) (end 146.05 58.42) (width 0.7) (layer "B.Cu") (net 9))
 (segment (start 90.17 100.615) (end 96.745 107.19) (width 0.7) (layer "B.Cu") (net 9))
 (segment (start 107.95 135.89) (end 109.38 134.46) (width 0.7) (layer "B.Cu") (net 9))
 (segment (start 109.38 134.46) (end 109.38 130.81) (width 0.7) (layer "B.Cu") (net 9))
 (segment (start 93.98 54.61) (end 90.17 58.42) (width 0.7) (layer "B.Cu") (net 9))
 (segment (start 104.14 116.84) (end 104.14 57.15) (width 0.7) (layer "B.Cu") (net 9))
 (segment (start 149.86 130.81) (end 149.86 135.89) (width 0.7) (layer "B.Cu") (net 9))
 (segment (start 101.49 88.125) (end 101.505 88.14) (width 0.7) (layer "B.Cu") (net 15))
 (segment (start 96.545 88.125) (end 101.49 88.125) (width 0.7) (layer "B.Cu") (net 15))
 (segment (start 96.745 112.27) (end 101.745 112.27) (width 0.7) (layer "B.Cu") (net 1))
 (segment (start 104.3 125.945) (end 104.3 130.81) (width 0.7) (layer "B.Cu") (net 12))
 (segment (start 144.78 130.81) (end 144.78 125.73) (width 0.7) (layer "B.Cu") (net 5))
 (segment (start 144.74 130.77) (end 144.78 130.81) (width 0.7) (layer "B.Cu") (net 5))
 (segment (start 151.13 106.68) (end 157.42 106.68) (width 0.7) (layer "B.Cu") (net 3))
 (segment (start 157.48 82.55) (end 151.19 82.55) (width 0.7) (layer "B.Cu") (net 18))
 (segment (start 157.48 62.23) (end 151.13 62.23) (width 0.7) (layer "B.Cu") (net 7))
 (segment (start 134.62 50.8) (end 137.16 48.26) (width 0.7) (layer "B.Cu") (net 23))
 (segment (start 134.62 53.34) (end 134.62 50.8) (width 0.7) (layer "B.Cu") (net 23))
 (segment (start 116.84 53.34) (end 119.38 53.34) (width 0.7) (layer "B.Cu") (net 19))
 (segment (start 114.3 50.8) (end 116.84 53.34) (width 0.7) (layer "B.Cu") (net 19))
 (segment (start 114.3 48.26) (end 114.3 50.8) (width 0.7) (layer "B.Cu") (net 19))
 (segment (start 119.38 55.88) (end 121.92 55.88) (width 0.7) (layer "B.Cu") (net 20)))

